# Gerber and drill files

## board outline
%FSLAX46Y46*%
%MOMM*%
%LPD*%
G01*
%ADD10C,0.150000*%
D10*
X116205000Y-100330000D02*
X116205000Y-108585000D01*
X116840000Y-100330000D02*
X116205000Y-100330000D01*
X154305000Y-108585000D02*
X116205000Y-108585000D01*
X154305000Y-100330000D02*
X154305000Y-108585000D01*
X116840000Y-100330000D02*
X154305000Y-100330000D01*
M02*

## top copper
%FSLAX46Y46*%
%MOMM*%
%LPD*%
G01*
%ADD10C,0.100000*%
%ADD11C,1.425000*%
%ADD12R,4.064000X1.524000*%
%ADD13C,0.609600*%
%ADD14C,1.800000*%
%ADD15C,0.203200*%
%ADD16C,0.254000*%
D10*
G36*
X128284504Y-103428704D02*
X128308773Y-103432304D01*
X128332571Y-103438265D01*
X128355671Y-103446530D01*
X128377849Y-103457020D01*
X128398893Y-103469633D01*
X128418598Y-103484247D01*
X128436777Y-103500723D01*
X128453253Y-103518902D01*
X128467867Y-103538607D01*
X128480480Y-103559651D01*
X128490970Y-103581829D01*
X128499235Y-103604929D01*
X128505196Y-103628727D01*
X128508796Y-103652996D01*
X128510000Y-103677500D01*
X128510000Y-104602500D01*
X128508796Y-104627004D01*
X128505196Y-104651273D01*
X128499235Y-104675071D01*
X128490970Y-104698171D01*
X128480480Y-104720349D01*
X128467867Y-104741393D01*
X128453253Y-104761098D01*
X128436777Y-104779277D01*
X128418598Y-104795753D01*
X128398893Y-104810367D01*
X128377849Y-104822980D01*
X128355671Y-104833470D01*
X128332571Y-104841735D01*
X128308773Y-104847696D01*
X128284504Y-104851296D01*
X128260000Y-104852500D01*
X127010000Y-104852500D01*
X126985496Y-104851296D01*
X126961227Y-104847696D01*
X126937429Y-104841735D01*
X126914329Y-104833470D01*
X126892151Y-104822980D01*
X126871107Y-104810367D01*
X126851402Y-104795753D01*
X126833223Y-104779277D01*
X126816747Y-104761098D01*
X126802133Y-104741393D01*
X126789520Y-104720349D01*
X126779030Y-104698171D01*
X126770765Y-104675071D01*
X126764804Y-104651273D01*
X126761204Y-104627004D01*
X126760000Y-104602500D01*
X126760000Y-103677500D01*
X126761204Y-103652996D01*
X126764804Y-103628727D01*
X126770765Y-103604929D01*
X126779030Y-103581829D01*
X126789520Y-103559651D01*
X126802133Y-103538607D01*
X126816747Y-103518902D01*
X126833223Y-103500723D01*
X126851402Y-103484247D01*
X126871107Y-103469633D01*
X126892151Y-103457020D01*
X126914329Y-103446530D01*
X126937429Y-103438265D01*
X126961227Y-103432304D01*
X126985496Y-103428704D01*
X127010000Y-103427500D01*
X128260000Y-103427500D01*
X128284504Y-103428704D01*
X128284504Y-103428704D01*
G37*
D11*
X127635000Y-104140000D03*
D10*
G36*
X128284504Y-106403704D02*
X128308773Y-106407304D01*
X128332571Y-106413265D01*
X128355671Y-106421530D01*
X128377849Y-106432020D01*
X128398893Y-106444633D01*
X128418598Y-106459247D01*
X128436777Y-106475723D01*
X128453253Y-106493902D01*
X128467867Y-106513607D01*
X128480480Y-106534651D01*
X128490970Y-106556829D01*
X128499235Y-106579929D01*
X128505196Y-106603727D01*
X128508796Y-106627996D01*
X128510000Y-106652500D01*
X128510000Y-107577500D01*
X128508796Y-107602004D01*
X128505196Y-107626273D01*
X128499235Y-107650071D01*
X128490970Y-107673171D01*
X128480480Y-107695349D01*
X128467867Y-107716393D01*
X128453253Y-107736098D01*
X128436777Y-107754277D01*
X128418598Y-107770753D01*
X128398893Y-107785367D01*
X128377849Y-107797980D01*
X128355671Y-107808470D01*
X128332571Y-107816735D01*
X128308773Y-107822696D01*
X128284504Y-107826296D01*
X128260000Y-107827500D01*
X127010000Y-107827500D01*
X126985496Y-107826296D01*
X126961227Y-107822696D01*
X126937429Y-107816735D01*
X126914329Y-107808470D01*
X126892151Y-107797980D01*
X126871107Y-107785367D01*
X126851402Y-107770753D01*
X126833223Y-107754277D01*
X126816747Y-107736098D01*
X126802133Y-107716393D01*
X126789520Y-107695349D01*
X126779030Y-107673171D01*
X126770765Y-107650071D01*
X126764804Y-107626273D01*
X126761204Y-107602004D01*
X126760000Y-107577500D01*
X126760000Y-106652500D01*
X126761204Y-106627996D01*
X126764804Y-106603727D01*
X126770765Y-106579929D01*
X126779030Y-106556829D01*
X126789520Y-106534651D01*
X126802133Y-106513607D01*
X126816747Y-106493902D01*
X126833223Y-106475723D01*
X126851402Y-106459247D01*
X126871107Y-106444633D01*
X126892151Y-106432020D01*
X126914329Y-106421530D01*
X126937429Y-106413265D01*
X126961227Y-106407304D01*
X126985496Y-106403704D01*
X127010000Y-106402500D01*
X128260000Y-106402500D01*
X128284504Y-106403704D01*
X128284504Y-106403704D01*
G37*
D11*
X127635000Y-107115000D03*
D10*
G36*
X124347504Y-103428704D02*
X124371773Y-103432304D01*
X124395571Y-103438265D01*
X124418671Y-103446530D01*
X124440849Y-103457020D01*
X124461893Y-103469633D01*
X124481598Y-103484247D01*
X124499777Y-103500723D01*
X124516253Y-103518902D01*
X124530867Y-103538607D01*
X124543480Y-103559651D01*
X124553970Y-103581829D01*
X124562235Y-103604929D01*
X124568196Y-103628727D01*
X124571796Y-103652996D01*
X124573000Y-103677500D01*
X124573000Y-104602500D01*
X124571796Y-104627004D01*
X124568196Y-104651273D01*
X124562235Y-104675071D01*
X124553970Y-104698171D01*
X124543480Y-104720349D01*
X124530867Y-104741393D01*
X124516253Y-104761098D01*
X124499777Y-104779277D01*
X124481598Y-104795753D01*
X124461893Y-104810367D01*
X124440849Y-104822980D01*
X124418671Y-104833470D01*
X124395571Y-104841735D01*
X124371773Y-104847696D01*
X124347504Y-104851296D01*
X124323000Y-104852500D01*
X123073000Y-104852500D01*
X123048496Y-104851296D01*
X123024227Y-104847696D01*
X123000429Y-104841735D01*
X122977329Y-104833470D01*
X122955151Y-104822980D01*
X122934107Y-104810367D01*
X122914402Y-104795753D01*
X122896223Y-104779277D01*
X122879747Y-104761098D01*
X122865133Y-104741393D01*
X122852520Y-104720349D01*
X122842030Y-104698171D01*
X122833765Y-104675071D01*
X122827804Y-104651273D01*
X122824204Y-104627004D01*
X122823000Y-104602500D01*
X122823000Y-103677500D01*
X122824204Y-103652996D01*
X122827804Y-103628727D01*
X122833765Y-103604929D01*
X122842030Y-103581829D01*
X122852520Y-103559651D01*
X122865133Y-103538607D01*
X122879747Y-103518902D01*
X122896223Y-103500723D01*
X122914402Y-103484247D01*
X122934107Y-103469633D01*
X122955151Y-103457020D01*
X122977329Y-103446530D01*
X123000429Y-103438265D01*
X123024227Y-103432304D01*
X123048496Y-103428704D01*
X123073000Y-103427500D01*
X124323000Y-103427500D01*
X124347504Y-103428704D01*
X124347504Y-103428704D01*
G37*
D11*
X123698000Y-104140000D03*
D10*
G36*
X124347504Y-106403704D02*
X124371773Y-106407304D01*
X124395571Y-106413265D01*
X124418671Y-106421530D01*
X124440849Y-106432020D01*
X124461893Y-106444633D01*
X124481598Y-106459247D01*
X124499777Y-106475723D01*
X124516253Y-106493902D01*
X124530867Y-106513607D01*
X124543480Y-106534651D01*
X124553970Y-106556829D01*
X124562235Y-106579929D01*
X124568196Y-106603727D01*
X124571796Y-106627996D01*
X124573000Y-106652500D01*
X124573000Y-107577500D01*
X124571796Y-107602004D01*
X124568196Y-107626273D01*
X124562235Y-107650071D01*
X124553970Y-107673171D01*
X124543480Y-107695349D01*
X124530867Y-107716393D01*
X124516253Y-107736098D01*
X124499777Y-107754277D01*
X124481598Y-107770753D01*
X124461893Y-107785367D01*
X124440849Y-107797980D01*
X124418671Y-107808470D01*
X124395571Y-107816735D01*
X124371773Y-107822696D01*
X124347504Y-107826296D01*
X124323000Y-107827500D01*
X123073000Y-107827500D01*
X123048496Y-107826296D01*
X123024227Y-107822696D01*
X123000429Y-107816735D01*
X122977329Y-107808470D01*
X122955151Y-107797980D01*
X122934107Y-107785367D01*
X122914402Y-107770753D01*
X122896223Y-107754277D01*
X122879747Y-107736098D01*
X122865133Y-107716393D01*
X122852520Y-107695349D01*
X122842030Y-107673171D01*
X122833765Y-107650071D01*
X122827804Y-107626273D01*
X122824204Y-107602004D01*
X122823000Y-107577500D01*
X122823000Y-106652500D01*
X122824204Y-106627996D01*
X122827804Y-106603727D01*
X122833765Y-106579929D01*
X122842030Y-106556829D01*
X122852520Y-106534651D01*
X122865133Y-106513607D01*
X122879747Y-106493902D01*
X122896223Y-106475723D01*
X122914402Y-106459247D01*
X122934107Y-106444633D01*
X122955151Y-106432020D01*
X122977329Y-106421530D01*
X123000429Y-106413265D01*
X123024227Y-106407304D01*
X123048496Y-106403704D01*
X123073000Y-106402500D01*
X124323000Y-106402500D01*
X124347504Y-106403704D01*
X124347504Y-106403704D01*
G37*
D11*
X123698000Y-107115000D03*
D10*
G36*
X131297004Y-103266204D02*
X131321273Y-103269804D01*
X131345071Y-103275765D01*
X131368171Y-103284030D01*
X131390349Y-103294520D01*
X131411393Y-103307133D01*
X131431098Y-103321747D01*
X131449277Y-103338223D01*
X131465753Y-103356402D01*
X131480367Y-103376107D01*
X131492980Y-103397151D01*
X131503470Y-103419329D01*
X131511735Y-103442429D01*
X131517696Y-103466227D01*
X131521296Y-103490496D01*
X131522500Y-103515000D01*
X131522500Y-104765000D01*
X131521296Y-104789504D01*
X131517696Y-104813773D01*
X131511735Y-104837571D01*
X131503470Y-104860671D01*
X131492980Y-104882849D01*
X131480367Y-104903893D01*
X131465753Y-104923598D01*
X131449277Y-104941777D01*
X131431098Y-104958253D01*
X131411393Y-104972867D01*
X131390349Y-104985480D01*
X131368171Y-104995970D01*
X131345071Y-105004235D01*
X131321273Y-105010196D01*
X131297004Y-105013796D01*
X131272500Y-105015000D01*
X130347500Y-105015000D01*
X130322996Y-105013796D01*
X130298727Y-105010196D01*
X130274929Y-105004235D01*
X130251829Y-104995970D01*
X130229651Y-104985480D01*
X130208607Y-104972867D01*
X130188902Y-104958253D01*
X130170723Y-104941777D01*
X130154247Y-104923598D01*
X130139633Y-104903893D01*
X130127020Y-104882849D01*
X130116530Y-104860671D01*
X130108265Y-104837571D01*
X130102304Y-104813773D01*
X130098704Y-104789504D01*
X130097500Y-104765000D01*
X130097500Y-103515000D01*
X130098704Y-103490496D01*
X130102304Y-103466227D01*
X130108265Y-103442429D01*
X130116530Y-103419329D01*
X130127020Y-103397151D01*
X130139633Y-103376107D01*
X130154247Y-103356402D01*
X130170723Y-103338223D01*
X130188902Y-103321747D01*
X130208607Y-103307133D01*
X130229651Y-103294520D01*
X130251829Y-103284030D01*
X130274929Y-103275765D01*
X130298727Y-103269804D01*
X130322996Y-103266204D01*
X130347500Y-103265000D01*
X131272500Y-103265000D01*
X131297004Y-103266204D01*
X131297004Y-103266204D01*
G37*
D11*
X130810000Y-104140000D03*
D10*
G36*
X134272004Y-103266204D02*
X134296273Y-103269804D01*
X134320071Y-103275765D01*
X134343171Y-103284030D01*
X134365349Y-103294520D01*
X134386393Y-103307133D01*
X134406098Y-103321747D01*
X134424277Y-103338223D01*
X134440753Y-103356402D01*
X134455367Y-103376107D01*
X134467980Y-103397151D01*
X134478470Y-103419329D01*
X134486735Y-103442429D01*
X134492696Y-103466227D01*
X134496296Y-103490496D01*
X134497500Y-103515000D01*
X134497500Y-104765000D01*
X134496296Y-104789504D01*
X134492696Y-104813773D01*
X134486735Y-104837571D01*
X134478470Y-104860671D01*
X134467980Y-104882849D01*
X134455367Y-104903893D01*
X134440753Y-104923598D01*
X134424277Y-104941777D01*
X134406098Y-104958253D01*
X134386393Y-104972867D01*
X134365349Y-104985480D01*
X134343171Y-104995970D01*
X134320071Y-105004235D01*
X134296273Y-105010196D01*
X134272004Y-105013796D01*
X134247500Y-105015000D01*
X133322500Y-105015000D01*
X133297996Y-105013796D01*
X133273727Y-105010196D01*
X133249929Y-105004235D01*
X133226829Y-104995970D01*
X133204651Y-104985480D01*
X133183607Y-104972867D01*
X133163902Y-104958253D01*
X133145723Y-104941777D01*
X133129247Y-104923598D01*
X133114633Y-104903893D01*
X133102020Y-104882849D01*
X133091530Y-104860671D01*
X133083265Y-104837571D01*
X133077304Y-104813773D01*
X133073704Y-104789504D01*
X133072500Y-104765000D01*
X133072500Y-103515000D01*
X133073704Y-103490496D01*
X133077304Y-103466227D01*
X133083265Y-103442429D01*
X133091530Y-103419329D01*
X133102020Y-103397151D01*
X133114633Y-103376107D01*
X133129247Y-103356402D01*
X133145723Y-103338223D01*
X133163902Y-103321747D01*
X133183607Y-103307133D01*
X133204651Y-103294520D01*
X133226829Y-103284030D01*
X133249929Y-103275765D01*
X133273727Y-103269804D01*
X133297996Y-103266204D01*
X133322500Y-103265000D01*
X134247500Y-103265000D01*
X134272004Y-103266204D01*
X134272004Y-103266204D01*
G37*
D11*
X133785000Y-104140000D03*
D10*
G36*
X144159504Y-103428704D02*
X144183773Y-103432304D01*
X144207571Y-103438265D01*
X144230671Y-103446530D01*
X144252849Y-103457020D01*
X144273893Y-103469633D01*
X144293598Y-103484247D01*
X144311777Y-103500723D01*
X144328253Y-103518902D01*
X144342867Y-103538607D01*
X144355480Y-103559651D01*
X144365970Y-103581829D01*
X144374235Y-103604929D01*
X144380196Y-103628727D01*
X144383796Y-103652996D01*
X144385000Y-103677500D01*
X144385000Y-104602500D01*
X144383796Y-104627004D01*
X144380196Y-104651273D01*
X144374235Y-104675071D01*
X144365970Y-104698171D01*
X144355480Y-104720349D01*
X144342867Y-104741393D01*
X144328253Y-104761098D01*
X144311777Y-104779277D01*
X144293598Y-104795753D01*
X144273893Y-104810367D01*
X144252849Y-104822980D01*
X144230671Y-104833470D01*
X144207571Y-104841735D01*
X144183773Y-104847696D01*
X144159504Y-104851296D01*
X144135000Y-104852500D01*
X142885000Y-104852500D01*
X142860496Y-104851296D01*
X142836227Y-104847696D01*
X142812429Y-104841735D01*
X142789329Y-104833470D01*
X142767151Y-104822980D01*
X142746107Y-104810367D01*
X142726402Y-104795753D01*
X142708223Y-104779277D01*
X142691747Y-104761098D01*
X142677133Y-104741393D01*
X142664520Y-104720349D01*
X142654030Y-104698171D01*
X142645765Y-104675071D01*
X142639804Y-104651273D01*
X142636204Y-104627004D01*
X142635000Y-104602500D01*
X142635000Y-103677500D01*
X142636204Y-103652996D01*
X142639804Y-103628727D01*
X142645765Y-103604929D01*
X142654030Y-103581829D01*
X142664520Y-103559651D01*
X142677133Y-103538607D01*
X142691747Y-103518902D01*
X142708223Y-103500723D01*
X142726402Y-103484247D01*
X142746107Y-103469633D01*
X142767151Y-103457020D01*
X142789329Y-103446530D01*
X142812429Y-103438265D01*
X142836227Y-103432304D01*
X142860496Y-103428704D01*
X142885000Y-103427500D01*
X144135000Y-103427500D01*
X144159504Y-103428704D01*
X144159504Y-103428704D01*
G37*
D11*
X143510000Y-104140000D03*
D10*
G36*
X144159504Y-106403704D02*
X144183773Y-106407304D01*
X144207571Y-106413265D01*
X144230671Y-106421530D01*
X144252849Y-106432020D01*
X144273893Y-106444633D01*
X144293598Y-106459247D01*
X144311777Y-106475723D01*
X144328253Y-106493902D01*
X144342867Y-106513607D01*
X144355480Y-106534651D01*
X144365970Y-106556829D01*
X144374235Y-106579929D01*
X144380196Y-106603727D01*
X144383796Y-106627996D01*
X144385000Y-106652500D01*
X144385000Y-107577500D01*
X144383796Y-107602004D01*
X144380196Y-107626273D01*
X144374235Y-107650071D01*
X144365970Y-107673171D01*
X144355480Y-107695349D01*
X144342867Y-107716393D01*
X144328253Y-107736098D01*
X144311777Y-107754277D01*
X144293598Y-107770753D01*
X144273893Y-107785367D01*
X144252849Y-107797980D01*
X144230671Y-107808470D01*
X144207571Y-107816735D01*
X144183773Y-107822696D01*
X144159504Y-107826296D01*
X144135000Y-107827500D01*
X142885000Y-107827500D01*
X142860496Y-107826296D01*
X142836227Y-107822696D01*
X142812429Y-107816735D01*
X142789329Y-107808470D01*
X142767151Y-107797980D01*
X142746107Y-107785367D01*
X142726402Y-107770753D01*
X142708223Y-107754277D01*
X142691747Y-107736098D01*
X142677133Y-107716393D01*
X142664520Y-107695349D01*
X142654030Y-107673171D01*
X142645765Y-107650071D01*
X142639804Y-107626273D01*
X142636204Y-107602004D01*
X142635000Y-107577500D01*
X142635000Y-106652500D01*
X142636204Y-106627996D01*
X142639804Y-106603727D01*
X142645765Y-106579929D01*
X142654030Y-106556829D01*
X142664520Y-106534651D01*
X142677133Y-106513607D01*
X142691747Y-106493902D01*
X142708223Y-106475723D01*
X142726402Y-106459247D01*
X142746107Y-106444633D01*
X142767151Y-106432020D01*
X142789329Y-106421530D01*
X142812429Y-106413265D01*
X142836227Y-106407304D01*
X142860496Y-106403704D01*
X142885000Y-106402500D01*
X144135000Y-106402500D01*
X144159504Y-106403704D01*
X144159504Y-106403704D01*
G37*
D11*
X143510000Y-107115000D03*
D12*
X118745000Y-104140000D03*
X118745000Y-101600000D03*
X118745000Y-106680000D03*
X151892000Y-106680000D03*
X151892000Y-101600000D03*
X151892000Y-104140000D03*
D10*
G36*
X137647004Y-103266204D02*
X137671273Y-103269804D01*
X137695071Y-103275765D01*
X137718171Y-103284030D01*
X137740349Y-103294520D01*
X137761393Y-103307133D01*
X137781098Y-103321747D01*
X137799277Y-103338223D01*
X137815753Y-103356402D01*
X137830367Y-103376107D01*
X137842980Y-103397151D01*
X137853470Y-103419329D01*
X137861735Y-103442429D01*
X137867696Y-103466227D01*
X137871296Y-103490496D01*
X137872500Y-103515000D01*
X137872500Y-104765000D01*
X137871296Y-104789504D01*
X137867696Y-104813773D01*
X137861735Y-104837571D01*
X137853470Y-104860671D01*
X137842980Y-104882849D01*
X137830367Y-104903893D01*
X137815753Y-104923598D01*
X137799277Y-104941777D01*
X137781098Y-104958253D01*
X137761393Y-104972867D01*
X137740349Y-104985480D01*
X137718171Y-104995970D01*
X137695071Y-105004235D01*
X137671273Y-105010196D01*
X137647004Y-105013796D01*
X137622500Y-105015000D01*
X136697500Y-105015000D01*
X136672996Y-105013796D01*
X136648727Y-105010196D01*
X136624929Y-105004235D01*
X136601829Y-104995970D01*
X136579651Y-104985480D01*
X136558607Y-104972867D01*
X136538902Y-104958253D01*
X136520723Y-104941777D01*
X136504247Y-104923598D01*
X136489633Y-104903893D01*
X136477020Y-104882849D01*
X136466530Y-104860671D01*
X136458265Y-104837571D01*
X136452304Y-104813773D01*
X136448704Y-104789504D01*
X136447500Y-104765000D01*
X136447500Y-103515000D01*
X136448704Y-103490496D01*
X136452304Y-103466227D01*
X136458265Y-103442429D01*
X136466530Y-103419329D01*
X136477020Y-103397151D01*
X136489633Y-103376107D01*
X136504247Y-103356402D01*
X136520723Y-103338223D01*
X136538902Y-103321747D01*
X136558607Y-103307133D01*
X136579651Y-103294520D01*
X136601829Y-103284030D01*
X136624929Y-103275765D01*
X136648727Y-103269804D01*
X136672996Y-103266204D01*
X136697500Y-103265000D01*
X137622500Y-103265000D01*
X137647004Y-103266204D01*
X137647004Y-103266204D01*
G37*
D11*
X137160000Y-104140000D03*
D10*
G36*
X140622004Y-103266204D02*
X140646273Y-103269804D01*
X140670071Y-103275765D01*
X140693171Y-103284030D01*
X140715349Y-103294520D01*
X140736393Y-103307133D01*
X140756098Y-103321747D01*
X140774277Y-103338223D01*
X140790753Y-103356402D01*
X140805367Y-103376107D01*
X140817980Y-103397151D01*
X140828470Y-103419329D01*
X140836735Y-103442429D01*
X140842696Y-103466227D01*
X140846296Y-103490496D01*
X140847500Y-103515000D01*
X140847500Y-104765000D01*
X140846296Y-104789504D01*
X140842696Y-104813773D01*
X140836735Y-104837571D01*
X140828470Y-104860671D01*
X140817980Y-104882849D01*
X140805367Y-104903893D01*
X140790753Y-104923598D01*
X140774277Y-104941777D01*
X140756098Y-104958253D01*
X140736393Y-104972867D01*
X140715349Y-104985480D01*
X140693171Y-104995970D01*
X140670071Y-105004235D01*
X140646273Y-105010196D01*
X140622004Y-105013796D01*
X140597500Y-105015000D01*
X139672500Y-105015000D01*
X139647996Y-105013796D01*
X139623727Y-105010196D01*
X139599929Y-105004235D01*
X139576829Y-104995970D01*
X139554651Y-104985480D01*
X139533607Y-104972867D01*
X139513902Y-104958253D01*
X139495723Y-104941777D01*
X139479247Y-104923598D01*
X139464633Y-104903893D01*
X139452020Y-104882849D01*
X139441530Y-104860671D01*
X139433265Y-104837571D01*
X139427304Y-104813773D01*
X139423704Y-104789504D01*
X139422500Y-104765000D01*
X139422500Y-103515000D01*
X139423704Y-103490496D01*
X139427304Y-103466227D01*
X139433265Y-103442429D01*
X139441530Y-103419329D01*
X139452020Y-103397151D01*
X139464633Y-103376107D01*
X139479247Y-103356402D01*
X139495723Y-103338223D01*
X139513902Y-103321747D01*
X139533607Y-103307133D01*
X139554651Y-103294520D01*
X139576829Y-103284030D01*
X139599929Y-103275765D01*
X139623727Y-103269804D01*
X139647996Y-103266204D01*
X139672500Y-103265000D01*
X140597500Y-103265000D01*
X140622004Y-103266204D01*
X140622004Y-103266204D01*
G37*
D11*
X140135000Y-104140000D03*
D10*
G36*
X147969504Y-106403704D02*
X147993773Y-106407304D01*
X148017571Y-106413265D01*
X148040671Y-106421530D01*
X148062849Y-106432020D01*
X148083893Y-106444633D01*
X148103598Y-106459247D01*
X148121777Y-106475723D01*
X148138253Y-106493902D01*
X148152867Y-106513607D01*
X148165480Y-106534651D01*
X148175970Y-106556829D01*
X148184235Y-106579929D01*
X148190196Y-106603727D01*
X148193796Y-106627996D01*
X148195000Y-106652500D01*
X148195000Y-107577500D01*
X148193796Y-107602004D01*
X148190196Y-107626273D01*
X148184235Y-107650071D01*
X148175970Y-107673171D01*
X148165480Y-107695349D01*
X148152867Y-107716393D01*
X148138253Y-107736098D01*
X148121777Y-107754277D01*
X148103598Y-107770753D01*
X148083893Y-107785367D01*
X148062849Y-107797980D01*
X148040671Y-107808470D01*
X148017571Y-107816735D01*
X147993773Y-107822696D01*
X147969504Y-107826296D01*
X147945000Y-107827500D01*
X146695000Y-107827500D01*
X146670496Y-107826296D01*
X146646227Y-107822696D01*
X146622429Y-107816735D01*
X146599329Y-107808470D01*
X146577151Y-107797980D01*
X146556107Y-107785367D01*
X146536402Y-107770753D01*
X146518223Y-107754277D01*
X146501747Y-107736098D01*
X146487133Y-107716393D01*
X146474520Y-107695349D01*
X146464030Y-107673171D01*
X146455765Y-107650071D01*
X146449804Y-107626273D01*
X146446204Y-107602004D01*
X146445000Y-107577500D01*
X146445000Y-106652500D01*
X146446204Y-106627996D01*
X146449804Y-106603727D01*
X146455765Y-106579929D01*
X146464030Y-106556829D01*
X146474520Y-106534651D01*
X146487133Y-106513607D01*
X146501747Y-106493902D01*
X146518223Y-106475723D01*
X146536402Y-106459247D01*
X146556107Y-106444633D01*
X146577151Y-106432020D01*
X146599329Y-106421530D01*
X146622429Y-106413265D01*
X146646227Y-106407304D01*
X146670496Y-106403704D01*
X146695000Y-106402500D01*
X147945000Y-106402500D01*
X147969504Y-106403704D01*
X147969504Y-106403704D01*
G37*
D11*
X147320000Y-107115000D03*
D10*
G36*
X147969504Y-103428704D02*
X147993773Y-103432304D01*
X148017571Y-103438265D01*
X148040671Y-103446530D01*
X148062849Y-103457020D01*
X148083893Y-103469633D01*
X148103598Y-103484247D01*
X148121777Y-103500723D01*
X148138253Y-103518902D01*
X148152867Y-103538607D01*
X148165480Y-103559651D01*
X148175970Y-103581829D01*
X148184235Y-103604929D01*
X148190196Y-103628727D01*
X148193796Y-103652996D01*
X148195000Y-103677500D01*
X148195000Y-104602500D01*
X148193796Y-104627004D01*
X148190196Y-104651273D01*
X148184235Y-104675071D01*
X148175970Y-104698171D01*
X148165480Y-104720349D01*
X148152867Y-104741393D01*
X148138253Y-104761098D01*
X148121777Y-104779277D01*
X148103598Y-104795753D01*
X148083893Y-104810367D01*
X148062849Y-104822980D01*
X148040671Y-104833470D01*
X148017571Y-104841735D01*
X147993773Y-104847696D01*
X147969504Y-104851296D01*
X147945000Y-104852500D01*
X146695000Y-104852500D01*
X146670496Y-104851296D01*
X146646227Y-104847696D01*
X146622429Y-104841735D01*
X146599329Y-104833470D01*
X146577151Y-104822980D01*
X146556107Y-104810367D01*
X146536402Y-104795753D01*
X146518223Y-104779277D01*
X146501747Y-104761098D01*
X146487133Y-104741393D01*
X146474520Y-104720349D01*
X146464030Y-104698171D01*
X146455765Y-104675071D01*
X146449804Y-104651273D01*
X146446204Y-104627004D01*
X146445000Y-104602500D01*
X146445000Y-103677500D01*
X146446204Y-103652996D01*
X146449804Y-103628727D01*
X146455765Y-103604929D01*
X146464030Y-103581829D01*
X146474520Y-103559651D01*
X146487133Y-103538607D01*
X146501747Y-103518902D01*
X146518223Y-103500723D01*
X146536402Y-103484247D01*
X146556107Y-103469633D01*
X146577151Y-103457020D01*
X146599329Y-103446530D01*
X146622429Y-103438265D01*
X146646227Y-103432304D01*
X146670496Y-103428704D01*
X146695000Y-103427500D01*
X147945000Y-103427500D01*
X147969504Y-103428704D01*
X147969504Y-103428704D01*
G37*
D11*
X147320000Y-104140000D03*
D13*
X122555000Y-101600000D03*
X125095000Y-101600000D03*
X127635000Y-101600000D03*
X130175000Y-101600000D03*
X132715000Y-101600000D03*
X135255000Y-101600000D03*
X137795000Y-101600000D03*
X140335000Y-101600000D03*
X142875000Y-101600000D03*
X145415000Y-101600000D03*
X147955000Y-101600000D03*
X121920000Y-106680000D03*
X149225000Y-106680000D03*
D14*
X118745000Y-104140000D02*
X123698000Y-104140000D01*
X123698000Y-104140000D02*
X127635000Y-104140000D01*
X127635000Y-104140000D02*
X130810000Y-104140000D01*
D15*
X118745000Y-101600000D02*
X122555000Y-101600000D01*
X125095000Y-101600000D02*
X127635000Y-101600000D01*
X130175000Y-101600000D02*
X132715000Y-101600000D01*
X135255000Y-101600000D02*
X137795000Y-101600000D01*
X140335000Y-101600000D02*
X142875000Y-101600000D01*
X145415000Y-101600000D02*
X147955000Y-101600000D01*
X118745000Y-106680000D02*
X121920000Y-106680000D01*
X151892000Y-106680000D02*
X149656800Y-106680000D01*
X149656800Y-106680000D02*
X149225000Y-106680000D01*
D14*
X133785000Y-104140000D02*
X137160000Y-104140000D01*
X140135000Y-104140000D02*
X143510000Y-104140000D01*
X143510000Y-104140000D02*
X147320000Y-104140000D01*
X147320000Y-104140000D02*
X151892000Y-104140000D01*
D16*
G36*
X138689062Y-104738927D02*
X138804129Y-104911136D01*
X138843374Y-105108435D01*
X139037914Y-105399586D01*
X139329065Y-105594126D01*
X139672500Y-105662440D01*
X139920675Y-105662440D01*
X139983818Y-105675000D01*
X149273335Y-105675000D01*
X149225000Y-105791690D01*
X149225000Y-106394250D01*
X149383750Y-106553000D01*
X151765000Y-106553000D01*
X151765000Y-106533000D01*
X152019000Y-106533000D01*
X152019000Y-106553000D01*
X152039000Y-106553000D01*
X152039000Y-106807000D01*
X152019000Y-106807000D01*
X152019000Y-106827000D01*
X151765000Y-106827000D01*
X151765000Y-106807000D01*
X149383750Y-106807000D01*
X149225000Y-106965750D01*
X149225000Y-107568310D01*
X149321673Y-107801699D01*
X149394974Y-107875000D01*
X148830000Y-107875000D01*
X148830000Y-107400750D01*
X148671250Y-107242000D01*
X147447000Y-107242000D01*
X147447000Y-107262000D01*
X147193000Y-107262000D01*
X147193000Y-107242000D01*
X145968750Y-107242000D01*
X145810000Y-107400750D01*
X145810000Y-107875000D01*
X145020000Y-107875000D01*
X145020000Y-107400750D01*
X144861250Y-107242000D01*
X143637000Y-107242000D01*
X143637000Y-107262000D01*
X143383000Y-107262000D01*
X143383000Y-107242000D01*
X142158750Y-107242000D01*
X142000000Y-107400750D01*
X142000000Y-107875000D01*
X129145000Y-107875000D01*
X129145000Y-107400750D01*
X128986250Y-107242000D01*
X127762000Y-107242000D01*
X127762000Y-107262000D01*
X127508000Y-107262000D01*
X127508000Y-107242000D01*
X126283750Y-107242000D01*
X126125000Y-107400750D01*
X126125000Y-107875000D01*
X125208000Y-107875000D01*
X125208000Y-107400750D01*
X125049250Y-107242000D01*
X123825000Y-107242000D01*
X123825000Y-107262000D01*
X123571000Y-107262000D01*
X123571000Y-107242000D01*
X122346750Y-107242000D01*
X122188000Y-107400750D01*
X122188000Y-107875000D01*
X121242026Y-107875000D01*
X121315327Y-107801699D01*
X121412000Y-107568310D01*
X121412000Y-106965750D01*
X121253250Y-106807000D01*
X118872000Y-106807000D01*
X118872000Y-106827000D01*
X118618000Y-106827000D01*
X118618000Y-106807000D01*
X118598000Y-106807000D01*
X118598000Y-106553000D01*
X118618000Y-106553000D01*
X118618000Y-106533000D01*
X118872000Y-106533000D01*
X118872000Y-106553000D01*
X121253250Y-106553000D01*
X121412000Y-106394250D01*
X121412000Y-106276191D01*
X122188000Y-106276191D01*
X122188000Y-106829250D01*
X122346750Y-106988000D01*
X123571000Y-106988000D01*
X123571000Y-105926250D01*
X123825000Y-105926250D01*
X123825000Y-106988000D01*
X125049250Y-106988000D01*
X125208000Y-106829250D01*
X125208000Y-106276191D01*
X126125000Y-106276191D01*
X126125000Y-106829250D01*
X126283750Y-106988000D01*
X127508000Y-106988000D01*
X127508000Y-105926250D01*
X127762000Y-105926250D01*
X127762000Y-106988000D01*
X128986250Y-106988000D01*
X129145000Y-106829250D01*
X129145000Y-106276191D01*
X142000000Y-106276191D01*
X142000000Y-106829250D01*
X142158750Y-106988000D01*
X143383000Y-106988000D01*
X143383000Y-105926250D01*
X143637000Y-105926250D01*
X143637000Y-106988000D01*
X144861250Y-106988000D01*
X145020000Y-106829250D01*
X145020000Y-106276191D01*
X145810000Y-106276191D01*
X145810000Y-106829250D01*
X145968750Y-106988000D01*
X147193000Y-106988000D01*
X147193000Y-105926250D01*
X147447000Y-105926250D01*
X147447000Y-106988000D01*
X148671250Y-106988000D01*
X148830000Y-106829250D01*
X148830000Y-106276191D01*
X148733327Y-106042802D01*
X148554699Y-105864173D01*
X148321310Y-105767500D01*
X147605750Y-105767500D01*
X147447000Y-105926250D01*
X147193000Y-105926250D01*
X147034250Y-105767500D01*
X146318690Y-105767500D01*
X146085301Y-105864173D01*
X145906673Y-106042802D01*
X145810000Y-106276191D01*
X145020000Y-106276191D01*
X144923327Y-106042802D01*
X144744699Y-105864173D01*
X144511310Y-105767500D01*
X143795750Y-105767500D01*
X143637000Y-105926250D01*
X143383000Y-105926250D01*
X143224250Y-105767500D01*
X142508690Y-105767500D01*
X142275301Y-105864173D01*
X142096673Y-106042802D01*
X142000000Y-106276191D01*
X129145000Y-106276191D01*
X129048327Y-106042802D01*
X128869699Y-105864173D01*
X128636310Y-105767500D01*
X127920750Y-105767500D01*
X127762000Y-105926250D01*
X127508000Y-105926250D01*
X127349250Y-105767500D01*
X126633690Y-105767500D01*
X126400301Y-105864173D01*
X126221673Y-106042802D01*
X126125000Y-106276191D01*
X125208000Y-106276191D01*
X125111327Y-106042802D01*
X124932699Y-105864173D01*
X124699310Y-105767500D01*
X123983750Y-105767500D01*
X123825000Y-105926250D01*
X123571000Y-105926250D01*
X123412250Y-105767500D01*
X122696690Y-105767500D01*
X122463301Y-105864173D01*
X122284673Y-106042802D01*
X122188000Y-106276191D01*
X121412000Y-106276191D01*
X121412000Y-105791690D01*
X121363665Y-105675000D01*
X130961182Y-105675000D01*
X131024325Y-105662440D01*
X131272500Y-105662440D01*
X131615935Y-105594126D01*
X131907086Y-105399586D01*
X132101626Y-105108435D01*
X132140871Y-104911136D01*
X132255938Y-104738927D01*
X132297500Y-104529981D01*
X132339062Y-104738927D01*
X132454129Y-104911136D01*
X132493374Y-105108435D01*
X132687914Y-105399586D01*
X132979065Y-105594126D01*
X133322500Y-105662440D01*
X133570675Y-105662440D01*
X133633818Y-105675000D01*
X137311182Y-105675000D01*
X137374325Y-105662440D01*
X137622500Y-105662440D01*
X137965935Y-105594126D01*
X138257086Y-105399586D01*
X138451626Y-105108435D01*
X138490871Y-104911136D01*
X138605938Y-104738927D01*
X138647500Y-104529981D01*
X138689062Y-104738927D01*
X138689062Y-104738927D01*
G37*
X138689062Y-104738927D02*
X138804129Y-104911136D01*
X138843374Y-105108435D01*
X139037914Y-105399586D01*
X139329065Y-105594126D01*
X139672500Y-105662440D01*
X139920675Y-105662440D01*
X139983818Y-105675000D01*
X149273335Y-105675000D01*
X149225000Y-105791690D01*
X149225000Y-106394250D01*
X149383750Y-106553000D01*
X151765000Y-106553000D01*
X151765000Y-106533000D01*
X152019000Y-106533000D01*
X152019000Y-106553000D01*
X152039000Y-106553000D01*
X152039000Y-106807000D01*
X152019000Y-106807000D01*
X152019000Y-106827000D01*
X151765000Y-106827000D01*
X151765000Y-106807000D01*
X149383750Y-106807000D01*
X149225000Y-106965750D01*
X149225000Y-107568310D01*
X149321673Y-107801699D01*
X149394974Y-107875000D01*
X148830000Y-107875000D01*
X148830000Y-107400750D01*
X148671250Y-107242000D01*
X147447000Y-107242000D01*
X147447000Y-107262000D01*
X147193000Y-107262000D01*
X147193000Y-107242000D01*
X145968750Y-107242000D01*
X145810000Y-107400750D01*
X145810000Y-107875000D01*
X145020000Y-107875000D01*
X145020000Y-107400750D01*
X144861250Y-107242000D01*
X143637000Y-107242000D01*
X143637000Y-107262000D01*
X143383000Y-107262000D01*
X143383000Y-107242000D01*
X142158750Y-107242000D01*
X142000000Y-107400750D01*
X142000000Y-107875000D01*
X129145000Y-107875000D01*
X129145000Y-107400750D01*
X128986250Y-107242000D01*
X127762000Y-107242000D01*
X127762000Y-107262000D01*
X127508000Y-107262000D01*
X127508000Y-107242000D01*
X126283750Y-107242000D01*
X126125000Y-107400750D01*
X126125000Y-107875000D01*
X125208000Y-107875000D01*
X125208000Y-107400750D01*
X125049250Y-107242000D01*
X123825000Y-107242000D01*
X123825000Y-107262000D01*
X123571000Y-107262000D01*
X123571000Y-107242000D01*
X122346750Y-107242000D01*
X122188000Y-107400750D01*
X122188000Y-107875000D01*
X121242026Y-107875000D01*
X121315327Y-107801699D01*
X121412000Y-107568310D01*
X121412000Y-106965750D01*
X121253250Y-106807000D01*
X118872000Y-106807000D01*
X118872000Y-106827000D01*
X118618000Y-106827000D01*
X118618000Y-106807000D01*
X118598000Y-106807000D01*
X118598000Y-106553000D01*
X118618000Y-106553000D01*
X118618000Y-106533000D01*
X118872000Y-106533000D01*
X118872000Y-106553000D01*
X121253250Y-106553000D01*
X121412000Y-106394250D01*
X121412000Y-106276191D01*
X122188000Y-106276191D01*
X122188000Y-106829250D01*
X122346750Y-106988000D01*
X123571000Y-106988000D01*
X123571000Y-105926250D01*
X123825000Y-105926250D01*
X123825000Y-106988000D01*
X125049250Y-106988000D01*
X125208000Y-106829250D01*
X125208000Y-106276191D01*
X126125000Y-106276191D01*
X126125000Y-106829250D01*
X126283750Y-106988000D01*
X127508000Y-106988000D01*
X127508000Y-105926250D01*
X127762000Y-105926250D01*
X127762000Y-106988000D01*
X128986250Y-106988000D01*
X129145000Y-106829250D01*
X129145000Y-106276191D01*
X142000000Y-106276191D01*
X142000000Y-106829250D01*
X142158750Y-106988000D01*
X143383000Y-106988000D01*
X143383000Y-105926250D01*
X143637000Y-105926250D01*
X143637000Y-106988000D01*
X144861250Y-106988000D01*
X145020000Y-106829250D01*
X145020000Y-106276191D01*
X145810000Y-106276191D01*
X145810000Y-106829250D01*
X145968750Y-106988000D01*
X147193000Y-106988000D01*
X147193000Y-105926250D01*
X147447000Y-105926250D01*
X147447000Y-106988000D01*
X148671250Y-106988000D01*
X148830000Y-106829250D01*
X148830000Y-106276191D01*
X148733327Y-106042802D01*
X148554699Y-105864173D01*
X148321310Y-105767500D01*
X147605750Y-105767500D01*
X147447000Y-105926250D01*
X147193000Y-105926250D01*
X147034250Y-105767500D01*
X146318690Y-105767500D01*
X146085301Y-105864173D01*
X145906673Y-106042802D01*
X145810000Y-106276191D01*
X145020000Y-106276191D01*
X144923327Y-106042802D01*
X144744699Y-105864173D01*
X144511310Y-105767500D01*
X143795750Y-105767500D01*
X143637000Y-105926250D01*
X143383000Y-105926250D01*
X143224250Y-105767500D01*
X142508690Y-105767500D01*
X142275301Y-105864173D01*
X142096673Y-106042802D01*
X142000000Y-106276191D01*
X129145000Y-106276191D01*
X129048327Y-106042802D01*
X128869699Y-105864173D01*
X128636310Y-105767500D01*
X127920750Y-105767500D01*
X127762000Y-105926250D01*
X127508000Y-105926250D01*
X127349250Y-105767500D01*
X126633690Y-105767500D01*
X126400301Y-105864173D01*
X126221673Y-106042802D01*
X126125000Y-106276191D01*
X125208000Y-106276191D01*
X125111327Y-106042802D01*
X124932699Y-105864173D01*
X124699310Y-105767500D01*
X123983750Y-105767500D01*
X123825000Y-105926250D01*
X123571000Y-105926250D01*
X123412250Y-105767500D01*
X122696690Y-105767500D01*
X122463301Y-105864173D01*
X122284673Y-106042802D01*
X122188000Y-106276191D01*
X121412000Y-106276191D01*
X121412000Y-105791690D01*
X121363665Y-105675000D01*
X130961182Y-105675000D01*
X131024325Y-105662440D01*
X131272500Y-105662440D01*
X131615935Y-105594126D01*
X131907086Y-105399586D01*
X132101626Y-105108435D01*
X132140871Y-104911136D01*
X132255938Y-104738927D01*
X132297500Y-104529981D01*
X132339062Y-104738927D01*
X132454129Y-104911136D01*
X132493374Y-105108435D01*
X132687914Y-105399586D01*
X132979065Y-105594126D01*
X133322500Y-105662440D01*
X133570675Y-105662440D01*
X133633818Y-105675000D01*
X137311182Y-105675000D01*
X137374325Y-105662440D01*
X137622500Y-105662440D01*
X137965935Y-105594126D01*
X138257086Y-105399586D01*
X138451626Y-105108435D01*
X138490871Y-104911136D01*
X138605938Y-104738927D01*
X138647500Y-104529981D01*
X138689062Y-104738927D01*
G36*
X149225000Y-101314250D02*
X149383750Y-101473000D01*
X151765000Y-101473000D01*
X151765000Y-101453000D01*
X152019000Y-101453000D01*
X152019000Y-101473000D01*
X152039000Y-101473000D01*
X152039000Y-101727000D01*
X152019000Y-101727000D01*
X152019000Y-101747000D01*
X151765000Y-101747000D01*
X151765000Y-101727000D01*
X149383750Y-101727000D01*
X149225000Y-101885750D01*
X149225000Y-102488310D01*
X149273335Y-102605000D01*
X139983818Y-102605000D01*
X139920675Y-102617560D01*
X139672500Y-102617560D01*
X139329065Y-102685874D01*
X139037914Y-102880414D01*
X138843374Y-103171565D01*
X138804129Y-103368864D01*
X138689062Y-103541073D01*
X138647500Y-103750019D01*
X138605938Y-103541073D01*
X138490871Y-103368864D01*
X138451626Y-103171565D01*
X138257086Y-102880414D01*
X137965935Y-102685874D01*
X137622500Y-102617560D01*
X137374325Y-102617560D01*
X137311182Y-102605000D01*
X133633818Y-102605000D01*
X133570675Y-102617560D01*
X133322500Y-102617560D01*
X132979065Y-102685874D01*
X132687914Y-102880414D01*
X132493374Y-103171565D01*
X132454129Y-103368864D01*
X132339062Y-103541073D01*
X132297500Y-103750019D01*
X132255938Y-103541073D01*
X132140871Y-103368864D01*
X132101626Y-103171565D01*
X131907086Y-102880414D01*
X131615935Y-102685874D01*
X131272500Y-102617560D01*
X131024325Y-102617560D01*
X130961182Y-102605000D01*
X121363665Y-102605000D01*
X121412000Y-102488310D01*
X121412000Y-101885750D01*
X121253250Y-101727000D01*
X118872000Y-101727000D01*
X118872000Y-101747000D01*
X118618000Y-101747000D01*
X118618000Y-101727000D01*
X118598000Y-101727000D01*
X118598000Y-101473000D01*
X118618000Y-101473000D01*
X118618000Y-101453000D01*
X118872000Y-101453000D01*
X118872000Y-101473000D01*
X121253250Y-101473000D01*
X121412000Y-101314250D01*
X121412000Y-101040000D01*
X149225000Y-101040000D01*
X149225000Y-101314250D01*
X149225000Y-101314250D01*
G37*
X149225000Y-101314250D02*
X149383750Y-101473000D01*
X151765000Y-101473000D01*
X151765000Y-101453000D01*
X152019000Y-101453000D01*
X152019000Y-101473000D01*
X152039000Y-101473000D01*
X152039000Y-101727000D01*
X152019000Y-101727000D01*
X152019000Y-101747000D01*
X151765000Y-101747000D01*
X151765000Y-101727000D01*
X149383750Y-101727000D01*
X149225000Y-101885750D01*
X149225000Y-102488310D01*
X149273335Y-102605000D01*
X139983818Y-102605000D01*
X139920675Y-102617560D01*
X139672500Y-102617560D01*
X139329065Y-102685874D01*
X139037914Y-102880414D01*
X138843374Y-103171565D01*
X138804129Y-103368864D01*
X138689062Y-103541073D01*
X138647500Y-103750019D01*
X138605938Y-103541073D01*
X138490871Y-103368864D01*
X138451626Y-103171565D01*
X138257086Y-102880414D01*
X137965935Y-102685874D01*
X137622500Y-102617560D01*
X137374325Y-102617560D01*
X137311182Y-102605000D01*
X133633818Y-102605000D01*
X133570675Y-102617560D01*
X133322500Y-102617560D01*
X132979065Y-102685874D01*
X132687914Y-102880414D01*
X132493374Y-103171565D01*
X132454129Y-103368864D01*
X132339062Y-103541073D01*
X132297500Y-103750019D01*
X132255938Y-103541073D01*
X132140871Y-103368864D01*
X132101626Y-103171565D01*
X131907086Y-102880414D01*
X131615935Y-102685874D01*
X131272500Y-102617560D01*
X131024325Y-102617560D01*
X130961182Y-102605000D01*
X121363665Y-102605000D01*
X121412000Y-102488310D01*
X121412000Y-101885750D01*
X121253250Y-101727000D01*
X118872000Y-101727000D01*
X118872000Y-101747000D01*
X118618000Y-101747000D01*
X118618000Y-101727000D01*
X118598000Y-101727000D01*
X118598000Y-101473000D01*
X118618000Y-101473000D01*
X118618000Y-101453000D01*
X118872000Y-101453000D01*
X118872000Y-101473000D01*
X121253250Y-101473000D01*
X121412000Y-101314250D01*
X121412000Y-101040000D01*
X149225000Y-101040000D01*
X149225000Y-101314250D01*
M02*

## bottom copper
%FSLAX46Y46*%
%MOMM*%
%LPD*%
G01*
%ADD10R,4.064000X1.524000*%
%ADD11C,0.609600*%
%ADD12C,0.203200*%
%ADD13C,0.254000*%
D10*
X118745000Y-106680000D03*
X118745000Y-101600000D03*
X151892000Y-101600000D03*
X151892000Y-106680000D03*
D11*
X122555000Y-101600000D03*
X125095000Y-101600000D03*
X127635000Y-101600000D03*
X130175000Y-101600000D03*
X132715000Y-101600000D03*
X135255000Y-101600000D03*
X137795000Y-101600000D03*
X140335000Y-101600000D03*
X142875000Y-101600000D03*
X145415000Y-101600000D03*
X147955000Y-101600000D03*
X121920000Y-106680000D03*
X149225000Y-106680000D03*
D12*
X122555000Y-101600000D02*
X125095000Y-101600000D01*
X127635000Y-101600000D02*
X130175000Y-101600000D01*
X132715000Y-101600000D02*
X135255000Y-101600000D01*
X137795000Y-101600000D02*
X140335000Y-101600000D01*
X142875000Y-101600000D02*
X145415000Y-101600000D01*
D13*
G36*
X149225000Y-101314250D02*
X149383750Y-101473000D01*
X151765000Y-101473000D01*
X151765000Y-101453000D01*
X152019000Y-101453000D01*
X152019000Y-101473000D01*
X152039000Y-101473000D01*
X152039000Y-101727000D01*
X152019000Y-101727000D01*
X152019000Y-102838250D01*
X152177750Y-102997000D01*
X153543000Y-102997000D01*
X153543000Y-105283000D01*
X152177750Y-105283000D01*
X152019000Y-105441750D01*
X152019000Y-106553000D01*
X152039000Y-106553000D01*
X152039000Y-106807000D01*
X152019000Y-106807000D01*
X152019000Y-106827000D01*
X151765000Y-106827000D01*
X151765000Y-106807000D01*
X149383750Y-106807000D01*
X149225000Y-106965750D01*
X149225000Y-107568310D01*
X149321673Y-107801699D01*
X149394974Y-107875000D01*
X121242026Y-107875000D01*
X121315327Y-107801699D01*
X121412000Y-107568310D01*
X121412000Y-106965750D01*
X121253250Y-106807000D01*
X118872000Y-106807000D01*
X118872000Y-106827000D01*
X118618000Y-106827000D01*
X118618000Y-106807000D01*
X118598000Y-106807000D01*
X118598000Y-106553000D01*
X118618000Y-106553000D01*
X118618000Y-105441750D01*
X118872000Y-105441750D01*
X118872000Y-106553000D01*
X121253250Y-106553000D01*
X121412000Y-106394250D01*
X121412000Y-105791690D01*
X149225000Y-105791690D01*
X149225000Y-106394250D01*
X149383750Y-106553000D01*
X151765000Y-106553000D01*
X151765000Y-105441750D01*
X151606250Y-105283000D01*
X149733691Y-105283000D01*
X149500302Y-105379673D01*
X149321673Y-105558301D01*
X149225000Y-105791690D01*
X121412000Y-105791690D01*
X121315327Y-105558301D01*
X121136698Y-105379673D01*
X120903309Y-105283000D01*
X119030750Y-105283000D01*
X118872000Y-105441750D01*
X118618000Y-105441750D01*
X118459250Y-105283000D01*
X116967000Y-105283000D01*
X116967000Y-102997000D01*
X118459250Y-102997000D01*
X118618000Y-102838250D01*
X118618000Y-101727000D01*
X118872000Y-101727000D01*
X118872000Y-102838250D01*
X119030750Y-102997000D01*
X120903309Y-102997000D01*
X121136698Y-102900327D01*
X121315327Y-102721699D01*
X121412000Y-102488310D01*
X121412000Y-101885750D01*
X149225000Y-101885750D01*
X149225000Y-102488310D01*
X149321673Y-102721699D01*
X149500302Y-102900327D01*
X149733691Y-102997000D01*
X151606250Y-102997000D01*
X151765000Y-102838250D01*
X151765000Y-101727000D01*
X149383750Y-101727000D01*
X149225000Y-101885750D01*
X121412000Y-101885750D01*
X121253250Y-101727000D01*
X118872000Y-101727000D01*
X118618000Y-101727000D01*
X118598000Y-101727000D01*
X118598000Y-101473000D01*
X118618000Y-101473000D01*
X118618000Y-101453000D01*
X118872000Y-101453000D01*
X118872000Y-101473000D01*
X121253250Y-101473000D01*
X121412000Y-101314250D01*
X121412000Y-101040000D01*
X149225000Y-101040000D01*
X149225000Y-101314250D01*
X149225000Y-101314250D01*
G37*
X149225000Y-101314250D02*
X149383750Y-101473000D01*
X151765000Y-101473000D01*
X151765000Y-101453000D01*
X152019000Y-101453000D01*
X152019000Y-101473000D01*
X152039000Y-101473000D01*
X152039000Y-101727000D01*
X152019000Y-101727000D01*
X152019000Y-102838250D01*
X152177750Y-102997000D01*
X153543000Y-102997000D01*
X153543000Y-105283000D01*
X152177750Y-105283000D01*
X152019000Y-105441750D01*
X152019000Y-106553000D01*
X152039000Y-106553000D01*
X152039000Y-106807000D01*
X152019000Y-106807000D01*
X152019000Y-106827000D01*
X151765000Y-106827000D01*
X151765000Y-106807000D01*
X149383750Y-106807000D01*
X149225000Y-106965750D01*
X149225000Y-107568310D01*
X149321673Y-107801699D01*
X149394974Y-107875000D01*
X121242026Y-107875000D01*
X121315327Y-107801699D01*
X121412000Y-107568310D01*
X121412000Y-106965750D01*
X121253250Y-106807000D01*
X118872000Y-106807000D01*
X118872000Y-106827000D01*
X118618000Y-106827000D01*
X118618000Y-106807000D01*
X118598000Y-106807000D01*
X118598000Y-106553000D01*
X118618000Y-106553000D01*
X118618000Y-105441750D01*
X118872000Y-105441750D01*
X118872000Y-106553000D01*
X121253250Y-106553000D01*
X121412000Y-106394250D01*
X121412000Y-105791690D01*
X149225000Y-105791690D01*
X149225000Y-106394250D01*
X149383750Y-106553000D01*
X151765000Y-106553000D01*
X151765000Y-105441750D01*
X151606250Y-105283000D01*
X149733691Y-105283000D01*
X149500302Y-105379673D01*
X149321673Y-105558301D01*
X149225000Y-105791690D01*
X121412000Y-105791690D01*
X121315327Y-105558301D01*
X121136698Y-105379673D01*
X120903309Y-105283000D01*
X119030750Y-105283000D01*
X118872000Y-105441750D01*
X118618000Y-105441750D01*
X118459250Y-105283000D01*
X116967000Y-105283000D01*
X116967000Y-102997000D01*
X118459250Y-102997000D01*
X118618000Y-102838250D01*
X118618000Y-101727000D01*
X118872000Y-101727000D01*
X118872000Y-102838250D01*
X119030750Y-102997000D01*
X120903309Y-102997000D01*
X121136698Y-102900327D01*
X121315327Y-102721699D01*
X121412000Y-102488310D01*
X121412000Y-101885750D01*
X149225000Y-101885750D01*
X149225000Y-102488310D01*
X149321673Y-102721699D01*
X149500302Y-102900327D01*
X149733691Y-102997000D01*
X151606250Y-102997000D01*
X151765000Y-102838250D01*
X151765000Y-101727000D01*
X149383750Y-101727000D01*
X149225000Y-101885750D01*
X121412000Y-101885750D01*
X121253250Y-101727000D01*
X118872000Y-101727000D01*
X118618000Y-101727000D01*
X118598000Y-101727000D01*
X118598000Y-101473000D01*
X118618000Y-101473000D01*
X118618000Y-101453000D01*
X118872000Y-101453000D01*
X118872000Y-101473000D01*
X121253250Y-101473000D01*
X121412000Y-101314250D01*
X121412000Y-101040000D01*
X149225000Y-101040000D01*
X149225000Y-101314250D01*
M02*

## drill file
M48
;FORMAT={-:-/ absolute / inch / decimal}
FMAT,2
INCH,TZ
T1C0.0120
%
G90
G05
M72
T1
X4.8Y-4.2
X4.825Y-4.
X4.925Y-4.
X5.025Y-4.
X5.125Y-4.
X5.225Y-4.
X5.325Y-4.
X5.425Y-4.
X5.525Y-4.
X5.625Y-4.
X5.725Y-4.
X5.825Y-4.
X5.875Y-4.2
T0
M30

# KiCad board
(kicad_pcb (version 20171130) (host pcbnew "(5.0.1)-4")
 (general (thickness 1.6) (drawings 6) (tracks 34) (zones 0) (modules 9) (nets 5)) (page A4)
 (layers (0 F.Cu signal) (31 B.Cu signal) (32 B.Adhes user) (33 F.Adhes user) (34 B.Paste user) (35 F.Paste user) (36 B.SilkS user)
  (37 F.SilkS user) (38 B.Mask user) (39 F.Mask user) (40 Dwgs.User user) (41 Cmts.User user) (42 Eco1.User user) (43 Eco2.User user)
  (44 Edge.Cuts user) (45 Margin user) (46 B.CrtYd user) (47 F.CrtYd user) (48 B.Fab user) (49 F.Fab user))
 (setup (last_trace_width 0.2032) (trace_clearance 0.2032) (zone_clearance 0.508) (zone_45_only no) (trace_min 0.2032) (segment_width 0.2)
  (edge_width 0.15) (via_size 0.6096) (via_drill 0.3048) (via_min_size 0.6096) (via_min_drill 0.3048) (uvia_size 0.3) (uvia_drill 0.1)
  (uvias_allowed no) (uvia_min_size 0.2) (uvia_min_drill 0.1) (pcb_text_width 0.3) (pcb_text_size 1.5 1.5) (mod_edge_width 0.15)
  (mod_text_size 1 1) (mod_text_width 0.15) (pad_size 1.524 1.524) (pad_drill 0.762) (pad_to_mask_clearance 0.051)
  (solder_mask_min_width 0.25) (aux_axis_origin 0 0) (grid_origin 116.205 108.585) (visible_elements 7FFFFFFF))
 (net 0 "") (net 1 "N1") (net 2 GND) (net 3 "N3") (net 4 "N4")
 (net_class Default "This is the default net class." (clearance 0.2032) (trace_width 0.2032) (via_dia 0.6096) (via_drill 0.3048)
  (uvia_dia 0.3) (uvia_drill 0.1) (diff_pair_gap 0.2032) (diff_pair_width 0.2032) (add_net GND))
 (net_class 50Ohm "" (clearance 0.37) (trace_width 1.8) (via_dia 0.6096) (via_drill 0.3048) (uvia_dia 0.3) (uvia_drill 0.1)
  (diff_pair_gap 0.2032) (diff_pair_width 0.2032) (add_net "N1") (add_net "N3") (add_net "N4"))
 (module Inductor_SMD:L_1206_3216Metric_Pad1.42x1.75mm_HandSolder (layer F.Cu) (at 127.635 105.6275 270)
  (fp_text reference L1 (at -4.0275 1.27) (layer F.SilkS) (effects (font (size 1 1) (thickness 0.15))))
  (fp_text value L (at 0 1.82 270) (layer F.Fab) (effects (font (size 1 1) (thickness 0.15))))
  (pad 1 smd roundrect (at -1.4875 0 270) (size 1.425 1.75) (layers F.Cu F.Paste F.Mask) (roundrect_rratio 0.175439) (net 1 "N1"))
  (pad 2 smd roundrect (at 1.4875 0 270) (size 1.425 1.75) (layers F.Cu F.Paste F.Mask) (roundrect_rratio 0.175439) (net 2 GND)))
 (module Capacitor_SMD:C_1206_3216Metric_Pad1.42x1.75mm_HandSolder (layer F.Cu) (at 123.698 105.6275 270)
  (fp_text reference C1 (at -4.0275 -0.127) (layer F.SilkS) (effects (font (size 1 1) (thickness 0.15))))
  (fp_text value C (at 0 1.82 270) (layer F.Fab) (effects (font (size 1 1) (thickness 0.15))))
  (pad 1 smd roundrect (at -1.4875 0 270) (size 1.425 1.75) (layers F.Cu F.Paste F.Mask) (roundrect_rratio 0.175439) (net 1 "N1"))
  (pad 2 smd roundrect (at 1.4875 0 270) (size 1.425 1.75) (layers F.Cu F.Paste F.Mask) (roundrect_rratio 0.175439) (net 2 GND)))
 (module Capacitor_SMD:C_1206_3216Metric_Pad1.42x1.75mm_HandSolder (layer F.Cu) (at 132.2975 104.14 180)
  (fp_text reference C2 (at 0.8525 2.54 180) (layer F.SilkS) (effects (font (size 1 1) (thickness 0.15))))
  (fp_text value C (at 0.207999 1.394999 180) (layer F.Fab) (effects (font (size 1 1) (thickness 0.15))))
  (pad 2 smd roundrect (at 1.4875 0 180) (size 1.425 1.75) (layers F.Cu F.Paste F.Mask) (roundrect_rratio 0.175439) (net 1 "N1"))
  (pad 1 smd roundrect (at -1.4875 0 180) (size 1.425 1.75) (layers F.Cu F.Paste F.Mask) (roundrect_rratio 0.175439) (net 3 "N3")))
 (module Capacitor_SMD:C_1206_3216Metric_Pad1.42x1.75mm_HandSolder (layer F.Cu) (at 143.51 105.6275 270)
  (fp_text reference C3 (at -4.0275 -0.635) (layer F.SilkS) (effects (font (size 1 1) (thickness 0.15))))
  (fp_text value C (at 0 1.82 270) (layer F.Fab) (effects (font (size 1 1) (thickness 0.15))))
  (pad 1 smd roundrect (at -1.4875 0 270) (size 1.425 1.75) (layers F.Cu F.Paste F.Mask) (roundrect_rratio 0.175439) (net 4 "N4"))
  (pad 2 smd roundrect (at 1.4875 0 270) (size 1.425 1.75) (layers F.Cu F.Paste F.Mask) (roundrect_rratio 0.175439) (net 2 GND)))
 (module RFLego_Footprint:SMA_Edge (layer F.Cu) (at 116.713 104.14)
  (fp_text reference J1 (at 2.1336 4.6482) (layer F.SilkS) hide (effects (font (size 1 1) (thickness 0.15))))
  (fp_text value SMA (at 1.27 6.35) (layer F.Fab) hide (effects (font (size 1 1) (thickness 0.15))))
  (pad 1 smd rect (at 2.032 0) (size 4.064 1.524) (layers F.Cu F.Mask) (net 1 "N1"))
  (pad 2 smd rect (at 2.032 -2.54) (size 4.064 1.524) (layers F.Cu F.Mask) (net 2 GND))
  (pad 2 smd rect (at 2.032 2.54) (size 4.064 1.524) (layers B.Cu B.Mask) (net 2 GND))
  (pad 2 smd rect (at 2.032 -2.54) (size 4.064 1.524) (layers B.Cu B.Mask) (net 2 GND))
  (pad 2 smd rect (at 2.032 2.54) (size 4.064 1.524) (layers F.Cu F.Mask) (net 2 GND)))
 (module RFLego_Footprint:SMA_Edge (layer F.Cu) (at 149.86 104.14)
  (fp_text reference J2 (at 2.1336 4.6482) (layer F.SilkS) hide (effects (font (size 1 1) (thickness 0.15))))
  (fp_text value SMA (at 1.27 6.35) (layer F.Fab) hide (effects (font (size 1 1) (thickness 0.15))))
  (pad 2 smd rect (at 2.032 2.54) (size 4.064 1.524) (layers F.Cu F.Mask) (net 2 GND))
  (pad 2 smd rect (at 2.032 -2.54) (size 4.064 1.524) (layers B.Cu B.Mask) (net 2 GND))
  (pad 2 smd rect (at 2.032 2.54) (size 4.064 1.524) (layers B.Cu B.Mask) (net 2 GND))
  (pad 2 smd rect (at 2.032 -2.54) (size 4.064 1.524) (layers F.Cu F.Mask) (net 2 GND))
  (pad 1 smd rect (at 2.032 0) (size 4.064 1.524) (layers F.Cu F.Mask) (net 4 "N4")))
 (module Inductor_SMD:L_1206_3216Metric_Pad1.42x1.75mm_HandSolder (layer F.Cu) (at 138.6475 104.14)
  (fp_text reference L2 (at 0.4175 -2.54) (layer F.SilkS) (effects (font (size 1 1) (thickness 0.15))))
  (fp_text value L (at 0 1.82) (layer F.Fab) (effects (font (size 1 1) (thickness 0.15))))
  (pad 1 smd roundrect (at -1.4875 0) (size 1.425 1.75) (layers F.Cu F.Paste F.Mask) (roundrect_rratio 0.175439) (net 3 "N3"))
  (pad 2 smd roundrect (at 1.4875 0) (size 1.425 1.75) (layers F.Cu F.Paste F.Mask) (roundrect_rratio 0.175439) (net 4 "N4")))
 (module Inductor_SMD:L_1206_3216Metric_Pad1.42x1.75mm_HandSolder (layer F.Cu) (at 147.32 105.6275 270)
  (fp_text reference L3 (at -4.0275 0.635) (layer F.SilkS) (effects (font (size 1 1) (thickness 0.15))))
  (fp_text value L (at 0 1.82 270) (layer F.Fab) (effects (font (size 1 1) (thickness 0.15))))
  (pad 2 smd roundrect (at 1.4875 0 270) (size 1.425 1.75) (layers F.Cu F.Paste F.Mask) (roundrect_rratio 0.175439) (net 2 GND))
  (pad 1 smd roundrect (at -1.4875 0 270) (size 1.425 1.75) (layers F.Cu F.Paste F.Mask) (roundrect_rratio 0.175439) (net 4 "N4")))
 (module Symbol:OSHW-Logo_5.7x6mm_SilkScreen (layer B.Cu) (at 126.365 104.775 180)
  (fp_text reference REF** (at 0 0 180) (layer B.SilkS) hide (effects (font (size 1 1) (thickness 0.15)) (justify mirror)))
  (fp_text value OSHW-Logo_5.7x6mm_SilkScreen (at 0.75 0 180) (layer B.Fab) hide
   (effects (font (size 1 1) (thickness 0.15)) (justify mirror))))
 (gr_line (start 116.205 100.33) (end 116.205 108.585) (layer Edge.Cuts) (width 0.15))
 (gr_line (start 116.84 100.33) (end 116.205 100.33) (layer Edge.Cuts) (width 0.15))
 (gr_line (start 154.305 108.585) (end 116.205 108.585) (layer Edge.Cuts) (width 0.15))
 (gr_line (start 154.305 100.33) (end 154.305 108.585) (layer Edge.Cuts) (width 0.15))
 (gr_line (start 116.84 100.33) (end 154.305 100.33) (layer Edge.Cuts) (width 0.15))
 (segment (start 118.745 104.14) (end 123.698 104.14) (width 1.8) (layer F.Cu) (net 1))
 (segment (start 123.698 104.14) (end 127.635 104.14) (width 1.8) (layer F.Cu) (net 1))
 (segment (start 127.635 104.14) (end 130.81 104.14) (width 1.8) (layer F.Cu) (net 1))
 (via (at 122.555 101.6) (size 0.6096) (drill 0.3048) (layers F.Cu B.Cu) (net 2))
 (segment (start 118.745 101.6) (end 122.555 101.6) (width 0.2032) (layer F.Cu) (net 2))
 (via (at 125.095 101.6) (size 0.6096) (drill 0.3048) (layers F.Cu B.Cu) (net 2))
 (segment (start 122.555 101.6) (end 125.095 101.6) (width 0.2032) (layer B.Cu) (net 2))
 (via (at 127.635 101.6) (size 0.6096) (drill 0.3048) (layers F.Cu B.Cu) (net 2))
 (segment (start 125.095 101.6) (end 127.635 101.6) (width 0.2032) (layer F.Cu) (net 2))
 (via (at 130.175 101.6) (size 0.6096) (drill 0.3048) (layers F.Cu B.Cu) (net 2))
 (segment (start 127.635 101.6) (end 130.175 101.6) (width 0.2032) (layer B.Cu) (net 2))
 (via (at 132.715 101.6) (size 0.6096) (drill 0.3048) (layers F.Cu B.Cu) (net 2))
 (segment (start 130.175 101.6) (end 132.715 101.6) (width 0.2032) (layer F.Cu) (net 2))
 (via (at 135.255 101.6) (size 0.6096) (drill 0.3048) (layers F.Cu B.Cu) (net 2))
 (segment (start 132.715 101.6) (end 135.255 101.6) (width 0.2032) (layer B.Cu) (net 2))
 (via (at 137.795 101.6) (size 0.6096) (drill 0.3048) (layers F.Cu B.Cu) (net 2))
 (segment (start 135.255 101.6) (end 137.795 101.6) (width 0.2032) (layer F.Cu) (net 2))
 (via (at 140.335 101.6) (size 0.6096) (drill 0.3048) (layers F.Cu B.Cu) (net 2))
 (segment (start 137.795 101.6) (end 140.335 101.6) (width 0.2032) (layer B.Cu) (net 2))
 (via (at 142.875 101.6) (size 0.6096) (drill 0.3048) (layers F.Cu B.Cu) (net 2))
 (segment (start 140.335 101.6) (end 142.875 101.6) (width 0.2032) (layer F.Cu) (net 2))
 (via (at 145.415 101.6) (size 0.6096) (drill 0.3048) (layers F.Cu B.Cu) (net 2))
 (segment (start 142.875 101.6) (end 145.415 101.6) (width 0.2032) (layer B.Cu) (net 2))
 (via (at 147.955 101.6) (size 0.6096) (drill 0.3048) (layers F.Cu B.Cu) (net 2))
 (segment (start 145.415 101.6) (end 147.955 101.6) (width 0.2032) (layer F.Cu) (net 2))
 (via (at 121.92 106.68) (size 0.6096) (drill 0.3048) (layers F.Cu B.Cu) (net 2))
 (segment (start 118.745 106.68) (end 121.92 106.68) (width 0.2032) (layer F.Cu) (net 2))
 (via (at 149.225 106.68) (size 0.6096) (drill 0.3048) (layers F.Cu B.Cu) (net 2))
 (segment (start 151.892 106.68) (end 149.6568 106.68) (width 0.2032) (layer F.Cu) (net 2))
 (segment (start 149.6568 106.68) (end 149.225 106.68) (width 0.2032) (layer F.Cu) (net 2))
 (segment (start 133.785 104.14) (end 137.16 104.14) (width 1.8) (layer F.Cu) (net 3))
 (segment (start 140.135 104.14) (end 143.51 104.14) (width 1.8) (layer F.Cu) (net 4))
 (segment (start 143.51 104.14) (end 147.32 104.14) (width 1.8) (layer F.Cu) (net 4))
 (segment (start 147.32 104.14) (end 151.892 104.14) (width 1.8) (layer F.Cu) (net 4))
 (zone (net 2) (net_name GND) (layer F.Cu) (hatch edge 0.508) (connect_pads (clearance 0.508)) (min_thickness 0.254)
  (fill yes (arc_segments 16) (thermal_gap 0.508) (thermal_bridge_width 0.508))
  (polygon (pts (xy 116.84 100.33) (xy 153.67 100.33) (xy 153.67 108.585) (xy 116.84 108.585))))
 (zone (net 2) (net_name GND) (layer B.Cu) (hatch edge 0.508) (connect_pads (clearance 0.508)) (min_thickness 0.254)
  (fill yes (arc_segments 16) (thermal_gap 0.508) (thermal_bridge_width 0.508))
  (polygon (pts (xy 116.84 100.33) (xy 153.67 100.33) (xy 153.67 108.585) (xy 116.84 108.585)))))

